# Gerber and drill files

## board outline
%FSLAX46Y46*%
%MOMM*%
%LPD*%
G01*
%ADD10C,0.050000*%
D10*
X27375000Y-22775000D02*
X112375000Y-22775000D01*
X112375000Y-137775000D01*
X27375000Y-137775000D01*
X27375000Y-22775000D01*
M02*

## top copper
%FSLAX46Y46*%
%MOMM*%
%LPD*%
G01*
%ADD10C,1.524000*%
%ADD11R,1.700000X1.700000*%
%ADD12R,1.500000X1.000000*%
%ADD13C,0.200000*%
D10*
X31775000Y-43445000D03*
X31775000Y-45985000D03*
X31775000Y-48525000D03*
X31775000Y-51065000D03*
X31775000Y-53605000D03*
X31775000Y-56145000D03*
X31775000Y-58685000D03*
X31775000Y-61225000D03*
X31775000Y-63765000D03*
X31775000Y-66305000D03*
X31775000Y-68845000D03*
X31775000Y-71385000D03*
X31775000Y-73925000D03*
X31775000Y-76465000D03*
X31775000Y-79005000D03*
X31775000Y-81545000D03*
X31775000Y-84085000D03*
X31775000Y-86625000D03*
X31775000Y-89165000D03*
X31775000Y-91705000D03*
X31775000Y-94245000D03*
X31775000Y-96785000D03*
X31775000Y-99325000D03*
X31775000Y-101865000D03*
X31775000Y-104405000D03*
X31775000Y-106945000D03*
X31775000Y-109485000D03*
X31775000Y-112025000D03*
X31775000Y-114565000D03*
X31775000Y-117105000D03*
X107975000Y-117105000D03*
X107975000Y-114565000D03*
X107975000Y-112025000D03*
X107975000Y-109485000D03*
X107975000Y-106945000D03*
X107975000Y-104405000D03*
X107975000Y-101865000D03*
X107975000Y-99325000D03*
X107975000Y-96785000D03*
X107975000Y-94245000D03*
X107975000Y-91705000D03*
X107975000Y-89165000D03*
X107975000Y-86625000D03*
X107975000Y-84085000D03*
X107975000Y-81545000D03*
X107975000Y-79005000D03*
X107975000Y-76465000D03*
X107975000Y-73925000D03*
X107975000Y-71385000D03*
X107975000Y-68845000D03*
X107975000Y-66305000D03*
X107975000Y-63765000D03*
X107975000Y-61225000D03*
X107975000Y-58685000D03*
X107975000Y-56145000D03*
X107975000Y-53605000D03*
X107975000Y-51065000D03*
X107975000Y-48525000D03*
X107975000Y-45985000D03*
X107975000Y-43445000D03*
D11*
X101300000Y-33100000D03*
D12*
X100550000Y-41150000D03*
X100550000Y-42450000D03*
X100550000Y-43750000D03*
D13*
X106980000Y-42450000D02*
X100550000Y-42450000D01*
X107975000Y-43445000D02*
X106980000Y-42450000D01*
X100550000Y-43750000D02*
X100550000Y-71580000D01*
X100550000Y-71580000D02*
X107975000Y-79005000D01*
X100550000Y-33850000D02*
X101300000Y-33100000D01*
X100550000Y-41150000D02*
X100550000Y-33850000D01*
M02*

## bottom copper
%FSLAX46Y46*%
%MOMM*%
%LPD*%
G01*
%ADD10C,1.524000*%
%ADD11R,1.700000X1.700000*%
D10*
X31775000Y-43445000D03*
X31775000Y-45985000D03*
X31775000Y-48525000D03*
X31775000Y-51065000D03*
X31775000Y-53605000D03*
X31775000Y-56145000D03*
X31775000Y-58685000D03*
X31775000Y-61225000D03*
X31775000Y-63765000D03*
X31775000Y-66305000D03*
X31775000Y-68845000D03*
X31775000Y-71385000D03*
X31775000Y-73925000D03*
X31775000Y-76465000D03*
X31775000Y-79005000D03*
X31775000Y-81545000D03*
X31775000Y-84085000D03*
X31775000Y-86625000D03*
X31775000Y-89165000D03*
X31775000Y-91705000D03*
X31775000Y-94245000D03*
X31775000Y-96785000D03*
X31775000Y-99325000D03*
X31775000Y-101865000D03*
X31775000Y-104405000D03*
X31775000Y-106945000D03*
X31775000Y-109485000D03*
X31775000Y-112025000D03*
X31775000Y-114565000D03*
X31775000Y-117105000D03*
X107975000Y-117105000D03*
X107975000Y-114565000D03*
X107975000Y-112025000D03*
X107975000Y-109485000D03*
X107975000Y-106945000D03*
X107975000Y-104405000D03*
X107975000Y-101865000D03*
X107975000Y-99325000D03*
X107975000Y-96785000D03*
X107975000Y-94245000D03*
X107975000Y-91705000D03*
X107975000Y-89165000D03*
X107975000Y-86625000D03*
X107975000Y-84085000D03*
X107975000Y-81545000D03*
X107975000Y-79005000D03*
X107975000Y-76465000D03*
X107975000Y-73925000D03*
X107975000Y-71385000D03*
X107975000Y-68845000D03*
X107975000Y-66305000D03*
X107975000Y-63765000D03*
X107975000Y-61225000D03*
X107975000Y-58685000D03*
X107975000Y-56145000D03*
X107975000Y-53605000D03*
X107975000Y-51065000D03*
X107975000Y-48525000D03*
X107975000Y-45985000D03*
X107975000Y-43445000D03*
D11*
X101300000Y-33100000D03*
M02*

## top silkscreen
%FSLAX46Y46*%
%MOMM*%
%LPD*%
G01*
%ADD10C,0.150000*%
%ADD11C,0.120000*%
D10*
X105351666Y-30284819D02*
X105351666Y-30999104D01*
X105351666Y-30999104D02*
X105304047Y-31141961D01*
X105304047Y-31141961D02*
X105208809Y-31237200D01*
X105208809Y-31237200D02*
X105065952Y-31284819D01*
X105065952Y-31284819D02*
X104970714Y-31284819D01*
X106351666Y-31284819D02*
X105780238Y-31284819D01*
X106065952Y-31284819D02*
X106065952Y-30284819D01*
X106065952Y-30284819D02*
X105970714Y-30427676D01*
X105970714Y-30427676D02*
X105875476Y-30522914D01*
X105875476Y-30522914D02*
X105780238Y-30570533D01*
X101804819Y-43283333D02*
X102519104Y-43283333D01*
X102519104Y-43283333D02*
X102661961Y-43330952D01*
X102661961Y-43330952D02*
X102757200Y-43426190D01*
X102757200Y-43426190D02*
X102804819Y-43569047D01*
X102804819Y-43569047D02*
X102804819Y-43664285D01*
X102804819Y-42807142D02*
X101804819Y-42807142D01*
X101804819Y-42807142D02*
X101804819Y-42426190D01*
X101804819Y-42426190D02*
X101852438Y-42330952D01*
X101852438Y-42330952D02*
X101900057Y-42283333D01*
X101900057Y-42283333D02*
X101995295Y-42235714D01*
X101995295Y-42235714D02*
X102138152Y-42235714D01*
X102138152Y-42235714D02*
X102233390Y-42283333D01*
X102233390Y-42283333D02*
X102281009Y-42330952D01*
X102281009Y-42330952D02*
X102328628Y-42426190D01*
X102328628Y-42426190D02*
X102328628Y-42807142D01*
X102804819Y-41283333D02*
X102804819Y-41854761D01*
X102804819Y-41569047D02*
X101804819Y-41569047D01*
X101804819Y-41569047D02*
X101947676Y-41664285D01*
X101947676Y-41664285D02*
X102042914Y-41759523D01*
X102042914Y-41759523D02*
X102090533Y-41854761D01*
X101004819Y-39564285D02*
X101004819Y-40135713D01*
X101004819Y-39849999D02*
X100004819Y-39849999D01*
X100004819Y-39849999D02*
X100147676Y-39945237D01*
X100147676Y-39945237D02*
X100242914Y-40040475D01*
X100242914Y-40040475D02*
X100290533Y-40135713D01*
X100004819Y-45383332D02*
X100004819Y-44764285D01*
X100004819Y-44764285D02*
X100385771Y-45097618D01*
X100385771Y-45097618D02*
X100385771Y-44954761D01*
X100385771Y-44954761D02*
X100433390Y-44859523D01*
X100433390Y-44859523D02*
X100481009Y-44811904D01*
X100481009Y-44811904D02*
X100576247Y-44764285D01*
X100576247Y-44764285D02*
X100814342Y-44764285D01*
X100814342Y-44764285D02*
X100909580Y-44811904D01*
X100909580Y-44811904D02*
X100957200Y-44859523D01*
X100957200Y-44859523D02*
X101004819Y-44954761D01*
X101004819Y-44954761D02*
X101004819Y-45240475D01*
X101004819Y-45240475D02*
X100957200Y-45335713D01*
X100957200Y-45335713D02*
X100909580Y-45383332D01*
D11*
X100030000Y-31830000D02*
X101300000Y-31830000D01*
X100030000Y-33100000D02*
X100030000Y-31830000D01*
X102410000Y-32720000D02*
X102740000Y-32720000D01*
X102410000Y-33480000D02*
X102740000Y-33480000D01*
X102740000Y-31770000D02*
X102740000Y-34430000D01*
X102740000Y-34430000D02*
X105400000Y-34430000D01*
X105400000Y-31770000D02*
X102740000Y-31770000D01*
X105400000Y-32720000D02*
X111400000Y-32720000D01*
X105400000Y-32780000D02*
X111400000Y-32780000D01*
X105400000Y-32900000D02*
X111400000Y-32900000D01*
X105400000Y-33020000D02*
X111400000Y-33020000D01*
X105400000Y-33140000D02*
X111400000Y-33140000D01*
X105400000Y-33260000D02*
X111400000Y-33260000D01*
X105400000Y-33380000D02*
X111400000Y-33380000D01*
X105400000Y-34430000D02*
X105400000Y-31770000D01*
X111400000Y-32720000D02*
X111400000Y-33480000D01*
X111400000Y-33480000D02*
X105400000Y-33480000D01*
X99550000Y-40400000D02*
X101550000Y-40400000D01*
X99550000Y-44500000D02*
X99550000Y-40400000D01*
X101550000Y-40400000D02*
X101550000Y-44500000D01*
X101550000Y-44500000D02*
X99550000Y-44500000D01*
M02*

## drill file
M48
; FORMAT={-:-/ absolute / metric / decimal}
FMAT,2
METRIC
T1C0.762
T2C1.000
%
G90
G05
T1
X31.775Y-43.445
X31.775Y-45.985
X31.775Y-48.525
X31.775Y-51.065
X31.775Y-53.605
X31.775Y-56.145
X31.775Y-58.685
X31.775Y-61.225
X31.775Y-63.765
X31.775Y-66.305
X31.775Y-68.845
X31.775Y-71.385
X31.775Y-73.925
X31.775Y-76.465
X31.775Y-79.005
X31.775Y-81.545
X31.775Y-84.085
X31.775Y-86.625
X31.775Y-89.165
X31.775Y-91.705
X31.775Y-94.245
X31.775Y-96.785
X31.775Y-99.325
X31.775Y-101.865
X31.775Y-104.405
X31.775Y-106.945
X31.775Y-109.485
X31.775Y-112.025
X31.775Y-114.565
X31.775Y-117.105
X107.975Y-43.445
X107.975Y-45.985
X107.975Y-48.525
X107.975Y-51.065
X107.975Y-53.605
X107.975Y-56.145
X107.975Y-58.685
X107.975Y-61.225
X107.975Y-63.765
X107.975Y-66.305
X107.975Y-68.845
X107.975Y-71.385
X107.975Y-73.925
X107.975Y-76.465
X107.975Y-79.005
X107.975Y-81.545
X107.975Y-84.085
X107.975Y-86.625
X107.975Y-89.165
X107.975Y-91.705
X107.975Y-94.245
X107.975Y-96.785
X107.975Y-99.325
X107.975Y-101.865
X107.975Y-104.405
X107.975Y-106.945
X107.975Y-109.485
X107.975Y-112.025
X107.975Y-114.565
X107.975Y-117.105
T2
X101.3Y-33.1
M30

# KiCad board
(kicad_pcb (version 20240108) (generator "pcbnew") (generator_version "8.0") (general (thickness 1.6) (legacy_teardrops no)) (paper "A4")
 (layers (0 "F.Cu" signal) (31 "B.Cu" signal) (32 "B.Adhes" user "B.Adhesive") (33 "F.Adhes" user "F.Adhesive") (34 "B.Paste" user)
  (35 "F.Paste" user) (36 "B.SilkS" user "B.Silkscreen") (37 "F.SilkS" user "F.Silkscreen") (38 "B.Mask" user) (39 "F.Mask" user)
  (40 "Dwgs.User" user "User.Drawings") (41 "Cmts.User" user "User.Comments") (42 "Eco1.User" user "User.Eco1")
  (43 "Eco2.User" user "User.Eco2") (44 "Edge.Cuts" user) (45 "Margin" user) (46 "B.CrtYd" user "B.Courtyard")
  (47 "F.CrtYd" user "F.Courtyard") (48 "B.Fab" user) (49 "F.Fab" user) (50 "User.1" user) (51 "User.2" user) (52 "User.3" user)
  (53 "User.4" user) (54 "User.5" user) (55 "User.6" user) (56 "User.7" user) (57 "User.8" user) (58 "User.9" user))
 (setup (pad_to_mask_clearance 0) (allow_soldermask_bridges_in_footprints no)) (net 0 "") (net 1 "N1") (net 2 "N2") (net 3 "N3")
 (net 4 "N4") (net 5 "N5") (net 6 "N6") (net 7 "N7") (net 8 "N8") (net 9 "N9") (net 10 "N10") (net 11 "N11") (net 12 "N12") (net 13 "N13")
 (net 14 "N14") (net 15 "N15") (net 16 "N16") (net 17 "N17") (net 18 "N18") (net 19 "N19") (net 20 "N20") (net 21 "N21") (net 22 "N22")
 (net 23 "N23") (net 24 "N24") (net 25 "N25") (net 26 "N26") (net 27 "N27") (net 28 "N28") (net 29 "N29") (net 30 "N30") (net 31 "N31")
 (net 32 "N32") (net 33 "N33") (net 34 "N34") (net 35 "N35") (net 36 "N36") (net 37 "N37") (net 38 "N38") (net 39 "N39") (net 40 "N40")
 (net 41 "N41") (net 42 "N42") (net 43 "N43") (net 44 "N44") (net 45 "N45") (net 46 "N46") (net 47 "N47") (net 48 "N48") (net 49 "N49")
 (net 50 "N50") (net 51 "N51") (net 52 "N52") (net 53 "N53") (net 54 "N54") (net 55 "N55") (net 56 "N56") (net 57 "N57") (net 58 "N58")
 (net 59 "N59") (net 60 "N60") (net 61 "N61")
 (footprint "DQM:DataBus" (layer "F.Cu") (at 71.575 79.745)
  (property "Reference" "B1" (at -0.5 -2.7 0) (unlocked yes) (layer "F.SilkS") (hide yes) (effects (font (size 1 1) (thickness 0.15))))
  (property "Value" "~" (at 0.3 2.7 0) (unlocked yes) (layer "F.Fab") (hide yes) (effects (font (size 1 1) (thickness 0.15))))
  (pad "1" thru_hole circle (at -39.8 -36.3) (size 1.524 1.524) (drill 0.762) (layers "*.Cu" "*.Mask") (remove_unused_layers no)
   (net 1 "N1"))
  (pad "2" thru_hole circle (at -39.8 -33.76) (size 1.524 1.524) (drill 0.762) (layers "*.Cu" "*.Mask") (remove_unused_layers no)
   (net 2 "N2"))
  (pad "3" thru_hole circle (at -39.8 -31.22) (size 1.524 1.524) (drill 0.762) (layers "*.Cu" "*.Mask") (remove_unused_layers no)
   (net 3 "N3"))
  (pad "4" thru_hole circle (at -39.8 -28.68) (size 1.524 1.524) (drill 0.762) (layers "*.Cu" "*.Mask") (remove_unused_layers no)
   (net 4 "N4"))
  (pad "5" thru_hole circle (at -39.8 -26.14) (size 1.524 1.524) (drill 0.762) (layers "*.Cu" "*.Mask") (remove_unused_layers no)
   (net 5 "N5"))
  (pad "6" thru_hole circle (at -39.8 -23.6) (size 1.524 1.524) (drill 0.762) (layers "*.Cu" "*.Mask") (remove_unused_layers no)
   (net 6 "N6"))
  (pad "7" thru_hole circle (at -39.8 -21.06) (size 1.524 1.524) (drill 0.762) (layers "*.Cu" "*.Mask") (remove_unused_layers no)
   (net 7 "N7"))
  (pad "8" thru_hole circle (at -39.8 -18.52) (size 1.524 1.524) (drill 0.762) (layers "*.Cu" "*.Mask") (remove_unused_layers no)
   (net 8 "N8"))
  (pad "9" thru_hole circle (at -39.8 -15.98) (size 1.524 1.524) (drill 0.762) (layers "*.Cu" "*.Mask") (remove_unused_layers no)
   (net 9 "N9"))
  (pad "10" thru_hole circle (at -39.8 -13.44) (size 1.524 1.524) (drill 0.762) (layers "*.Cu" "*.Mask") (remove_unused_layers no)
   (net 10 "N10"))
  (pad "11" thru_hole circle (at -39.8 -10.9) (size 1.524 1.524) (drill 0.762) (layers "*.Cu" "*.Mask") (remove_unused_layers no)
   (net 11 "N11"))
  (pad "12" thru_hole circle (at -39.8 -8.36) (size 1.524 1.524) (drill 0.762) (layers "*.Cu" "*.Mask") (remove_unused_layers no)
   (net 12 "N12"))
  (pad "13" thru_hole circle (at -39.8 -5.82) (size 1.524 1.524) (drill 0.762) (layers "*.Cu" "*.Mask") (remove_unused_layers no)
   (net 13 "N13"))
  (pad "14" thru_hole circle (at -39.8 -3.28) (size 1.524 1.524) (drill 0.762) (layers "*.Cu" "*.Mask") (remove_unused_layers no)
   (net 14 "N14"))
  (pad "15" thru_hole circle (at -39.8 -0.74) (size 1.524 1.524) (drill 0.762) (layers "*.Cu" "*.Mask") (remove_unused_layers no)
   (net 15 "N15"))
  (pad "16" thru_hole circle (at -39.8 1.8) (size 1.524 1.524) (drill 0.762) (layers "*.Cu" "*.Mask") (remove_unused_layers no)
   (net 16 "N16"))
  (pad "17" thru_hole circle (at -39.8 4.34) (size 1.524 1.524) (drill 0.762) (layers "*.Cu" "*.Mask") (remove_unused_layers no)
   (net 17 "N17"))
  (pad "18" thru_hole circle (at -39.8 6.88) (size 1.524 1.524) (drill 0.762) (layers "*.Cu" "*.Mask") (remove_unused_layers no)
   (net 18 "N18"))
  (pad "19" thru_hole circle (at -39.8 9.42) (size 1.524 1.524) (drill 0.762) (layers "*.Cu" "*.Mask") (remove_unused_layers no)
   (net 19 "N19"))
  (pad "20" thru_hole circle (at -39.8 11.96) (size 1.524 1.524) (drill 0.762) (layers "*.Cu" "*.Mask") (remove_unused_layers no)
   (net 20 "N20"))
  (pad "21" thru_hole circle (at -39.8 14.5) (size 1.524 1.524) (drill 0.762) (layers "*.Cu" "*.Mask") (remove_unused_layers no)
   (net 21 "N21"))
  (pad "22" thru_hole circle (at -39.8 17.04) (size 1.524 1.524) (drill 0.762) (layers "*.Cu" "*.Mask") (remove_unused_layers no)
   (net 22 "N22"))
  (pad "23" thru_hole circle (at -39.8 19.58) (size 1.524 1.524) (drill 0.762) (layers "*.Cu" "*.Mask") (remove_unused_layers no)
   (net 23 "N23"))
  (pad "24" thru_hole circle (at -39.8 22.12) (size 1.524 1.524) (drill 0.762) (layers "*.Cu" "*.Mask") (remove_unused_layers no)
   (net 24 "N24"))
  (pad "25" thru_hole circle (at -39.8 24.66) (size 1.524 1.524) (drill 0.762) (layers "*.Cu" "*.Mask") (remove_unused_layers no)
   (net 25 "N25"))
  (pad "26" thru_hole circle (at -39.8 27.2) (size 1.524 1.524) (drill 0.762) (layers "*.Cu" "*.Mask") (remove_unused_layers no)
   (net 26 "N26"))
  (pad "27" thru_hole circle (at -39.8 29.74) (size 1.524 1.524) (drill 0.762) (layers "*.Cu" "*.Mask") (remove_unused_layers no)
   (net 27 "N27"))
  (pad "28" thru_hole circle (at -39.8 32.28) (size 1.524 1.524) (drill 0.762) (layers "*.Cu" "*.Mask") (remove_unused_layers no)
   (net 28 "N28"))
  (pad "29" thru_hole circle (at -39.8 34.82) (size 1.524 1.524) (drill 0.762) (layers "*.Cu" "*.Mask") (remove_unused_layers no)
   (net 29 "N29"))
  (pad "30" thru_hole circle (at -39.8 37.36) (size 1.524 1.524) (drill 0.762) (layers "*.Cu" "*.Mask") (remove_unused_layers no)
   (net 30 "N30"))
  (pad "31" thru_hole circle (at 36.4 37.36) (size 1.524 1.524) (drill 0.762) (layers "*.Cu" "*.Mask") (remove_unused_layers no)
   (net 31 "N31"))
  (pad "32" thru_hole circle (at 36.4 34.82) (size 1.524 1.524) (drill 0.762) (layers "*.Cu" "*.Mask") (remove_unused_layers no)
   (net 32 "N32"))
  (pad "33" thru_hole circle (at 36.4 32.28) (size 1.524 1.524) (drill 0.762) (layers "*.Cu" "*.Mask") (remove_unused_layers no)
   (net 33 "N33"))
  (pad "34" thru_hole circle (at 36.4 29.74) (size 1.524 1.524) (drill 0.762) (layers "*.Cu" "*.Mask") (remove_unused_layers no)
   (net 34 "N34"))
  (pad "35" thru_hole circle (at 36.4 27.2) (size 1.524 1.524) (drill 0.762) (layers "*.Cu" "*.Mask") (remove_unused_layers no)
   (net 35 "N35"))
  (pad "36" thru_hole circle (at 36.4 24.66) (size 1.524 1.524) (drill 0.762) (layers "*.Cu" "*.Mask") (remove_unused_layers no)
   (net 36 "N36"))
  (pad "37" thru_hole circle (at 36.4 22.12) (size 1.524 1.524) (drill 0.762) (layers "*.Cu" "*.Mask") (remove_unused_layers no)
   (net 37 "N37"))
  (pad "38" thru_hole circle (at 36.4 19.58) (size 1.524 1.524) (drill 0.762) (layers "*.Cu" "*.Mask") (remove_unused_layers no)
   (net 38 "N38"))
  (pad "39" thru_hole circle (at 36.4 17.04) (size 1.524 1.524) (drill 0.762) (layers "*.Cu" "*.Mask") (remove_unused_layers no)
   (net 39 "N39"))
  (pad "40" thru_hole circle (at 36.4 14.5) (size 1.524 1.524) (drill 0.762) (layers "*.Cu" "*.Mask") (remove_unused_layers no)
   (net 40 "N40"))
  (pad "41" thru_hole circle (at 36.4 11.96) (size 1.524 1.524) (drill 0.762) (layers "*.Cu" "*.Mask") (remove_unused_layers no)
   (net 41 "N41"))
  (pad "42" thru_hole circle (at 36.4 9.42) (size 1.524 1.524) (drill 0.762) (layers "*.Cu" "*.Mask") (remove_unused_layers no)
   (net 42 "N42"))
  (pad "43" thru_hole circle (at 36.4 6.88) (size 1.524 1.524) (drill 0.762) (layers "*.Cu" "*.Mask") (remove_unused_layers no)
   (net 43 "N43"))
  (pad "44" thru_hole circle (at 36.4 4.34) (size 1.524 1.524) (drill 0.762) (layers "*.Cu" "*.Mask") (remove_unused_layers no)
   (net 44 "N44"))
  (pad "45" thru_hole circle (at 36.4 1.8) (size 1.524 1.524) (drill 0.762) (layers "*.Cu" "*.Mask") (remove_unused_layers no)
   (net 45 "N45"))
  (pad "46" thru_hole circle (at 36.4 -0.74) (size 1.524 1.524) (drill 0.762) (layers "*.Cu" "*.Mask") (remove_unused_layers no)
   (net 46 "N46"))
  (pad "47" thru_hole circle (at 36.4 -3.28) (size 1.524 1.524) (drill 0.762) (layers "*.Cu" "*.Mask") (remove_unused_layers no)
   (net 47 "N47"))
  (pad "48" thru_hole circle (at 36.4 -5.82) (size 1.524 1.524) (drill 0.762) (layers "*.Cu" "*.Mask") (remove_unused_layers no)
   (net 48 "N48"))
  (pad "49" thru_hole circle (at 36.4 -8.36) (size 1.524 1.524) (drill 0.762) (layers "*.Cu" "*.Mask") (remove_unused_layers no)
   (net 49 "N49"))
  (pad "50" thru_hole circle (at 36.4 -10.9) (size 1.524 1.524) (drill 0.762) (layers "*.Cu" "*.Mask") (remove_unused_layers no)
   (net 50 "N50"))
  (pad "51" thru_hole circle (at 36.4 -13.44) (size 1.524 1.524) (drill 0.762) (layers "*.Cu" "*.Mask") (remove_unused_layers no)
   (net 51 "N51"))
  (pad "52" thru_hole circle (at 36.4 -15.98) (size 1.524 1.524) (drill 0.762) (layers "*.Cu" "*.Mask") (remove_unused_layers no)
   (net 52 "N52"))
  (pad "53" thru_hole circle (at 36.4 -18.52) (size 1.524 1.524) (drill 0.762) (layers "*.Cu" "*.Mask") (remove_unused_layers no)
   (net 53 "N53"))
  (pad "54" thru_hole circle (at 36.4 -21.06) (size 1.524 1.524) (drill 0.762) (layers "*.Cu" "*.Mask") (remove_unused_layers no)
   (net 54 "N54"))
  (pad "55" thru_hole circle (at 36.4 -23.6) (size 1.524 1.524) (drill 0.762) (layers "*.Cu" "*.Mask") (remove_unused_layers no)
   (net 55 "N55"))
  (pad "56" thru_hole circle (at 36.4 -26.14) (size 1.524 1.524) (drill 0.762) (layers "*.Cu" "*.Mask") (remove_unused_layers no)
   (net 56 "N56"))
  (pad "57" thru_hole circle (at 36.4 -28.68) (size 1.524 1.524) (drill 0.762) (layers "*.Cu" "*.Mask") (remove_unused_layers no)
   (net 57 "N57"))
  (pad "58" thru_hole circle (at 36.4 -31.22) (size 1.524 1.524) (drill 0.762) (layers "*.Cu" "*.Mask") (remove_unused_layers no)
   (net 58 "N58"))
  (pad "59" thru_hole circle (at 36.4 -33.76) (size 1.524 1.524) (drill 0.762) (layers "*.Cu" "*.Mask") (remove_unused_layers no)
   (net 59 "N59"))
  (pad "60" thru_hole circle (at 36.4 -36.3) (size 1.524 1.524) (drill 0.762) (layers "*.Cu" "*.Mask") (remove_unused_layers no)
   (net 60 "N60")))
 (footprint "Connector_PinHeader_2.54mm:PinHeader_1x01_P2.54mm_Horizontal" (layer "F.Cu") (at 101.3 33.1)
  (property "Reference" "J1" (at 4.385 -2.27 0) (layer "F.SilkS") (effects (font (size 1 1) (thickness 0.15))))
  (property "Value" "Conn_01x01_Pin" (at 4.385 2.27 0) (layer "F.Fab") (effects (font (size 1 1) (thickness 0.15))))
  (fp_line (start -1.27 -1.27) (end 0 -1.27) (stroke (width 0.12) (type solid)) (layer "F.SilkS"))
  (fp_line (start -1.27 0) (end -1.27 -1.27) (stroke (width 0.12) (type solid)) (layer "F.SilkS"))
  (fp_line (start 1.11 -0.38) (end 1.44 -0.38) (stroke (width 0.12) (type solid)) (layer "F.SilkS"))
  (fp_line (start 1.11 0.38) (end 1.44 0.38) (stroke (width 0.12) (type solid)) (layer "F.SilkS"))
  (fp_line (start 1.44 -1.33) (end 1.44 1.33) (stroke (width 0.12) (type solid)) (layer "F.SilkS"))
  (fp_line (start 1.44 1.33) (end 4.1 1.33) (stroke (width 0.12) (type solid)) (layer "F.SilkS"))
  (fp_line (start 4.1 -1.33) (end 1.44 -1.33) (stroke (width 0.12) (type solid)) (layer "F.SilkS"))
  (fp_line (start 4.1 -0.38) (end 10.1 -0.38) (stroke (width 0.12) (type solid)) (layer "F.SilkS"))
  (fp_line (start 4.1 -0.32) (end 10.1 -0.32) (stroke (width 0.12) (type solid)) (layer "F.SilkS"))
  (fp_line (start 4.1 -0.2) (end 10.1 -0.2) (stroke (width 0.12) (type solid)) (layer "F.SilkS"))
  (fp_line (start 4.1 -0.08) (end 10.1 -0.08) (stroke (width 0.12) (type solid)) (layer "F.SilkS"))
  (fp_line (start 4.1 0.04) (end 10.1 0.04) (stroke (width 0.12) (type solid)) (layer "F.SilkS"))
  (fp_line (start 4.1 0.16) (end 10.1 0.16) (stroke (width 0.12) (type solid)) (layer "F.SilkS"))
  (fp_line (start 4.1 0.28) (end 10.1 0.28) (stroke (width 0.12) (type solid)) (layer "F.SilkS"))
  (fp_line (start 4.1 1.33) (end 4.1 -1.33) (stroke (width 0.12) (type solid)) (layer "F.SilkS"))
  (fp_line (start 10.1 -0.38) (end 10.1 0.38) (stroke (width 0.12) (type solid)) (layer "F.SilkS"))
  (fp_line (start 10.1 0.38) (end 4.1 0.38) (stroke (width 0.12) (type solid)) (layer "F.SilkS"))
  (pad "1" thru_hole rect (at 0 0) (size 1.7 1.7) (drill 1) (layers "*.Cu" "*.Mask") (remove_unused_layers no) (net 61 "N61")))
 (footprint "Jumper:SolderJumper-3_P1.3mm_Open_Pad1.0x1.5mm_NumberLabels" (layer "F.Cu") (at 100.55 42.45 -90)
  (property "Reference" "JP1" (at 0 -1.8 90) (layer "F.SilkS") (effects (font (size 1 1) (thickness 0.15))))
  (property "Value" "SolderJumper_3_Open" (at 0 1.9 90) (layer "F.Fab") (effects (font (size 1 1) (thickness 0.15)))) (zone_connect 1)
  (fp_line (start -2.05 1) (end -2.05 -1) (stroke (width 0.12) (type solid)) (layer "F.SilkS"))
  (fp_line (start 2.05 1) (end -2.05 1) (stroke (width 0.12) (type solid)) (layer "F.SilkS"))
  (fp_line (start -2.05 -1) (end 2.05 -1) (stroke (width 0.12) (type solid)) (layer "F.SilkS"))
  (fp_line (start 2.05 -1) (end 2.05 1) (stroke (width 0.12) (type solid)) (layer "F.SilkS"))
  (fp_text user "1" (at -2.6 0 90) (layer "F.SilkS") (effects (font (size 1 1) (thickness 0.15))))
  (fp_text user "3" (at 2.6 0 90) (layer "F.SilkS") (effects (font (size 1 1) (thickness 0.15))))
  (pad "1" smd rect (at -1.3 0 270) (size 1 1.5) (layers "F.Cu" "F.Mask") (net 61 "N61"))
  (pad "2" smd rect (at 0 0 270) (size 1 1.5) (layers "F.Cu" "F.Mask") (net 60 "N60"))
  (pad "3" smd rect (at 1.3 0 270) (size 1 1.5) (layers "F.Cu" "F.Mask") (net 46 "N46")))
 (gr_rect (start 27.375 22.775) (end 112.375 137.775) (stroke (width 0.05) (type default)) (fill none) (layer "Edge.Cuts"))
 (segment (start 106.98 42.45) (end 100.55 42.45) (width 0.2) (layer "F.Cu") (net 60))
 (segment (start 107.975 43.445) (end 106.98 42.45) (width 0.2) (layer "F.Cu") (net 60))
 (segment (start 100.55 43.75) (end 100.55 71.58) (width 0.2) (layer "F.Cu") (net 46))
 (segment (start 100.55 71.58) (end 107.975 79.005) (width 0.2) (layer "F.Cu") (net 46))
 (segment (start 100.55 33.85) (end 101.3 33.1) (width 0.2) (layer "F.Cu") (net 61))
 (segment (start 100.55 41.15) (end 100.55 33.85) (width 0.2) (layer "F.Cu") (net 61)))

